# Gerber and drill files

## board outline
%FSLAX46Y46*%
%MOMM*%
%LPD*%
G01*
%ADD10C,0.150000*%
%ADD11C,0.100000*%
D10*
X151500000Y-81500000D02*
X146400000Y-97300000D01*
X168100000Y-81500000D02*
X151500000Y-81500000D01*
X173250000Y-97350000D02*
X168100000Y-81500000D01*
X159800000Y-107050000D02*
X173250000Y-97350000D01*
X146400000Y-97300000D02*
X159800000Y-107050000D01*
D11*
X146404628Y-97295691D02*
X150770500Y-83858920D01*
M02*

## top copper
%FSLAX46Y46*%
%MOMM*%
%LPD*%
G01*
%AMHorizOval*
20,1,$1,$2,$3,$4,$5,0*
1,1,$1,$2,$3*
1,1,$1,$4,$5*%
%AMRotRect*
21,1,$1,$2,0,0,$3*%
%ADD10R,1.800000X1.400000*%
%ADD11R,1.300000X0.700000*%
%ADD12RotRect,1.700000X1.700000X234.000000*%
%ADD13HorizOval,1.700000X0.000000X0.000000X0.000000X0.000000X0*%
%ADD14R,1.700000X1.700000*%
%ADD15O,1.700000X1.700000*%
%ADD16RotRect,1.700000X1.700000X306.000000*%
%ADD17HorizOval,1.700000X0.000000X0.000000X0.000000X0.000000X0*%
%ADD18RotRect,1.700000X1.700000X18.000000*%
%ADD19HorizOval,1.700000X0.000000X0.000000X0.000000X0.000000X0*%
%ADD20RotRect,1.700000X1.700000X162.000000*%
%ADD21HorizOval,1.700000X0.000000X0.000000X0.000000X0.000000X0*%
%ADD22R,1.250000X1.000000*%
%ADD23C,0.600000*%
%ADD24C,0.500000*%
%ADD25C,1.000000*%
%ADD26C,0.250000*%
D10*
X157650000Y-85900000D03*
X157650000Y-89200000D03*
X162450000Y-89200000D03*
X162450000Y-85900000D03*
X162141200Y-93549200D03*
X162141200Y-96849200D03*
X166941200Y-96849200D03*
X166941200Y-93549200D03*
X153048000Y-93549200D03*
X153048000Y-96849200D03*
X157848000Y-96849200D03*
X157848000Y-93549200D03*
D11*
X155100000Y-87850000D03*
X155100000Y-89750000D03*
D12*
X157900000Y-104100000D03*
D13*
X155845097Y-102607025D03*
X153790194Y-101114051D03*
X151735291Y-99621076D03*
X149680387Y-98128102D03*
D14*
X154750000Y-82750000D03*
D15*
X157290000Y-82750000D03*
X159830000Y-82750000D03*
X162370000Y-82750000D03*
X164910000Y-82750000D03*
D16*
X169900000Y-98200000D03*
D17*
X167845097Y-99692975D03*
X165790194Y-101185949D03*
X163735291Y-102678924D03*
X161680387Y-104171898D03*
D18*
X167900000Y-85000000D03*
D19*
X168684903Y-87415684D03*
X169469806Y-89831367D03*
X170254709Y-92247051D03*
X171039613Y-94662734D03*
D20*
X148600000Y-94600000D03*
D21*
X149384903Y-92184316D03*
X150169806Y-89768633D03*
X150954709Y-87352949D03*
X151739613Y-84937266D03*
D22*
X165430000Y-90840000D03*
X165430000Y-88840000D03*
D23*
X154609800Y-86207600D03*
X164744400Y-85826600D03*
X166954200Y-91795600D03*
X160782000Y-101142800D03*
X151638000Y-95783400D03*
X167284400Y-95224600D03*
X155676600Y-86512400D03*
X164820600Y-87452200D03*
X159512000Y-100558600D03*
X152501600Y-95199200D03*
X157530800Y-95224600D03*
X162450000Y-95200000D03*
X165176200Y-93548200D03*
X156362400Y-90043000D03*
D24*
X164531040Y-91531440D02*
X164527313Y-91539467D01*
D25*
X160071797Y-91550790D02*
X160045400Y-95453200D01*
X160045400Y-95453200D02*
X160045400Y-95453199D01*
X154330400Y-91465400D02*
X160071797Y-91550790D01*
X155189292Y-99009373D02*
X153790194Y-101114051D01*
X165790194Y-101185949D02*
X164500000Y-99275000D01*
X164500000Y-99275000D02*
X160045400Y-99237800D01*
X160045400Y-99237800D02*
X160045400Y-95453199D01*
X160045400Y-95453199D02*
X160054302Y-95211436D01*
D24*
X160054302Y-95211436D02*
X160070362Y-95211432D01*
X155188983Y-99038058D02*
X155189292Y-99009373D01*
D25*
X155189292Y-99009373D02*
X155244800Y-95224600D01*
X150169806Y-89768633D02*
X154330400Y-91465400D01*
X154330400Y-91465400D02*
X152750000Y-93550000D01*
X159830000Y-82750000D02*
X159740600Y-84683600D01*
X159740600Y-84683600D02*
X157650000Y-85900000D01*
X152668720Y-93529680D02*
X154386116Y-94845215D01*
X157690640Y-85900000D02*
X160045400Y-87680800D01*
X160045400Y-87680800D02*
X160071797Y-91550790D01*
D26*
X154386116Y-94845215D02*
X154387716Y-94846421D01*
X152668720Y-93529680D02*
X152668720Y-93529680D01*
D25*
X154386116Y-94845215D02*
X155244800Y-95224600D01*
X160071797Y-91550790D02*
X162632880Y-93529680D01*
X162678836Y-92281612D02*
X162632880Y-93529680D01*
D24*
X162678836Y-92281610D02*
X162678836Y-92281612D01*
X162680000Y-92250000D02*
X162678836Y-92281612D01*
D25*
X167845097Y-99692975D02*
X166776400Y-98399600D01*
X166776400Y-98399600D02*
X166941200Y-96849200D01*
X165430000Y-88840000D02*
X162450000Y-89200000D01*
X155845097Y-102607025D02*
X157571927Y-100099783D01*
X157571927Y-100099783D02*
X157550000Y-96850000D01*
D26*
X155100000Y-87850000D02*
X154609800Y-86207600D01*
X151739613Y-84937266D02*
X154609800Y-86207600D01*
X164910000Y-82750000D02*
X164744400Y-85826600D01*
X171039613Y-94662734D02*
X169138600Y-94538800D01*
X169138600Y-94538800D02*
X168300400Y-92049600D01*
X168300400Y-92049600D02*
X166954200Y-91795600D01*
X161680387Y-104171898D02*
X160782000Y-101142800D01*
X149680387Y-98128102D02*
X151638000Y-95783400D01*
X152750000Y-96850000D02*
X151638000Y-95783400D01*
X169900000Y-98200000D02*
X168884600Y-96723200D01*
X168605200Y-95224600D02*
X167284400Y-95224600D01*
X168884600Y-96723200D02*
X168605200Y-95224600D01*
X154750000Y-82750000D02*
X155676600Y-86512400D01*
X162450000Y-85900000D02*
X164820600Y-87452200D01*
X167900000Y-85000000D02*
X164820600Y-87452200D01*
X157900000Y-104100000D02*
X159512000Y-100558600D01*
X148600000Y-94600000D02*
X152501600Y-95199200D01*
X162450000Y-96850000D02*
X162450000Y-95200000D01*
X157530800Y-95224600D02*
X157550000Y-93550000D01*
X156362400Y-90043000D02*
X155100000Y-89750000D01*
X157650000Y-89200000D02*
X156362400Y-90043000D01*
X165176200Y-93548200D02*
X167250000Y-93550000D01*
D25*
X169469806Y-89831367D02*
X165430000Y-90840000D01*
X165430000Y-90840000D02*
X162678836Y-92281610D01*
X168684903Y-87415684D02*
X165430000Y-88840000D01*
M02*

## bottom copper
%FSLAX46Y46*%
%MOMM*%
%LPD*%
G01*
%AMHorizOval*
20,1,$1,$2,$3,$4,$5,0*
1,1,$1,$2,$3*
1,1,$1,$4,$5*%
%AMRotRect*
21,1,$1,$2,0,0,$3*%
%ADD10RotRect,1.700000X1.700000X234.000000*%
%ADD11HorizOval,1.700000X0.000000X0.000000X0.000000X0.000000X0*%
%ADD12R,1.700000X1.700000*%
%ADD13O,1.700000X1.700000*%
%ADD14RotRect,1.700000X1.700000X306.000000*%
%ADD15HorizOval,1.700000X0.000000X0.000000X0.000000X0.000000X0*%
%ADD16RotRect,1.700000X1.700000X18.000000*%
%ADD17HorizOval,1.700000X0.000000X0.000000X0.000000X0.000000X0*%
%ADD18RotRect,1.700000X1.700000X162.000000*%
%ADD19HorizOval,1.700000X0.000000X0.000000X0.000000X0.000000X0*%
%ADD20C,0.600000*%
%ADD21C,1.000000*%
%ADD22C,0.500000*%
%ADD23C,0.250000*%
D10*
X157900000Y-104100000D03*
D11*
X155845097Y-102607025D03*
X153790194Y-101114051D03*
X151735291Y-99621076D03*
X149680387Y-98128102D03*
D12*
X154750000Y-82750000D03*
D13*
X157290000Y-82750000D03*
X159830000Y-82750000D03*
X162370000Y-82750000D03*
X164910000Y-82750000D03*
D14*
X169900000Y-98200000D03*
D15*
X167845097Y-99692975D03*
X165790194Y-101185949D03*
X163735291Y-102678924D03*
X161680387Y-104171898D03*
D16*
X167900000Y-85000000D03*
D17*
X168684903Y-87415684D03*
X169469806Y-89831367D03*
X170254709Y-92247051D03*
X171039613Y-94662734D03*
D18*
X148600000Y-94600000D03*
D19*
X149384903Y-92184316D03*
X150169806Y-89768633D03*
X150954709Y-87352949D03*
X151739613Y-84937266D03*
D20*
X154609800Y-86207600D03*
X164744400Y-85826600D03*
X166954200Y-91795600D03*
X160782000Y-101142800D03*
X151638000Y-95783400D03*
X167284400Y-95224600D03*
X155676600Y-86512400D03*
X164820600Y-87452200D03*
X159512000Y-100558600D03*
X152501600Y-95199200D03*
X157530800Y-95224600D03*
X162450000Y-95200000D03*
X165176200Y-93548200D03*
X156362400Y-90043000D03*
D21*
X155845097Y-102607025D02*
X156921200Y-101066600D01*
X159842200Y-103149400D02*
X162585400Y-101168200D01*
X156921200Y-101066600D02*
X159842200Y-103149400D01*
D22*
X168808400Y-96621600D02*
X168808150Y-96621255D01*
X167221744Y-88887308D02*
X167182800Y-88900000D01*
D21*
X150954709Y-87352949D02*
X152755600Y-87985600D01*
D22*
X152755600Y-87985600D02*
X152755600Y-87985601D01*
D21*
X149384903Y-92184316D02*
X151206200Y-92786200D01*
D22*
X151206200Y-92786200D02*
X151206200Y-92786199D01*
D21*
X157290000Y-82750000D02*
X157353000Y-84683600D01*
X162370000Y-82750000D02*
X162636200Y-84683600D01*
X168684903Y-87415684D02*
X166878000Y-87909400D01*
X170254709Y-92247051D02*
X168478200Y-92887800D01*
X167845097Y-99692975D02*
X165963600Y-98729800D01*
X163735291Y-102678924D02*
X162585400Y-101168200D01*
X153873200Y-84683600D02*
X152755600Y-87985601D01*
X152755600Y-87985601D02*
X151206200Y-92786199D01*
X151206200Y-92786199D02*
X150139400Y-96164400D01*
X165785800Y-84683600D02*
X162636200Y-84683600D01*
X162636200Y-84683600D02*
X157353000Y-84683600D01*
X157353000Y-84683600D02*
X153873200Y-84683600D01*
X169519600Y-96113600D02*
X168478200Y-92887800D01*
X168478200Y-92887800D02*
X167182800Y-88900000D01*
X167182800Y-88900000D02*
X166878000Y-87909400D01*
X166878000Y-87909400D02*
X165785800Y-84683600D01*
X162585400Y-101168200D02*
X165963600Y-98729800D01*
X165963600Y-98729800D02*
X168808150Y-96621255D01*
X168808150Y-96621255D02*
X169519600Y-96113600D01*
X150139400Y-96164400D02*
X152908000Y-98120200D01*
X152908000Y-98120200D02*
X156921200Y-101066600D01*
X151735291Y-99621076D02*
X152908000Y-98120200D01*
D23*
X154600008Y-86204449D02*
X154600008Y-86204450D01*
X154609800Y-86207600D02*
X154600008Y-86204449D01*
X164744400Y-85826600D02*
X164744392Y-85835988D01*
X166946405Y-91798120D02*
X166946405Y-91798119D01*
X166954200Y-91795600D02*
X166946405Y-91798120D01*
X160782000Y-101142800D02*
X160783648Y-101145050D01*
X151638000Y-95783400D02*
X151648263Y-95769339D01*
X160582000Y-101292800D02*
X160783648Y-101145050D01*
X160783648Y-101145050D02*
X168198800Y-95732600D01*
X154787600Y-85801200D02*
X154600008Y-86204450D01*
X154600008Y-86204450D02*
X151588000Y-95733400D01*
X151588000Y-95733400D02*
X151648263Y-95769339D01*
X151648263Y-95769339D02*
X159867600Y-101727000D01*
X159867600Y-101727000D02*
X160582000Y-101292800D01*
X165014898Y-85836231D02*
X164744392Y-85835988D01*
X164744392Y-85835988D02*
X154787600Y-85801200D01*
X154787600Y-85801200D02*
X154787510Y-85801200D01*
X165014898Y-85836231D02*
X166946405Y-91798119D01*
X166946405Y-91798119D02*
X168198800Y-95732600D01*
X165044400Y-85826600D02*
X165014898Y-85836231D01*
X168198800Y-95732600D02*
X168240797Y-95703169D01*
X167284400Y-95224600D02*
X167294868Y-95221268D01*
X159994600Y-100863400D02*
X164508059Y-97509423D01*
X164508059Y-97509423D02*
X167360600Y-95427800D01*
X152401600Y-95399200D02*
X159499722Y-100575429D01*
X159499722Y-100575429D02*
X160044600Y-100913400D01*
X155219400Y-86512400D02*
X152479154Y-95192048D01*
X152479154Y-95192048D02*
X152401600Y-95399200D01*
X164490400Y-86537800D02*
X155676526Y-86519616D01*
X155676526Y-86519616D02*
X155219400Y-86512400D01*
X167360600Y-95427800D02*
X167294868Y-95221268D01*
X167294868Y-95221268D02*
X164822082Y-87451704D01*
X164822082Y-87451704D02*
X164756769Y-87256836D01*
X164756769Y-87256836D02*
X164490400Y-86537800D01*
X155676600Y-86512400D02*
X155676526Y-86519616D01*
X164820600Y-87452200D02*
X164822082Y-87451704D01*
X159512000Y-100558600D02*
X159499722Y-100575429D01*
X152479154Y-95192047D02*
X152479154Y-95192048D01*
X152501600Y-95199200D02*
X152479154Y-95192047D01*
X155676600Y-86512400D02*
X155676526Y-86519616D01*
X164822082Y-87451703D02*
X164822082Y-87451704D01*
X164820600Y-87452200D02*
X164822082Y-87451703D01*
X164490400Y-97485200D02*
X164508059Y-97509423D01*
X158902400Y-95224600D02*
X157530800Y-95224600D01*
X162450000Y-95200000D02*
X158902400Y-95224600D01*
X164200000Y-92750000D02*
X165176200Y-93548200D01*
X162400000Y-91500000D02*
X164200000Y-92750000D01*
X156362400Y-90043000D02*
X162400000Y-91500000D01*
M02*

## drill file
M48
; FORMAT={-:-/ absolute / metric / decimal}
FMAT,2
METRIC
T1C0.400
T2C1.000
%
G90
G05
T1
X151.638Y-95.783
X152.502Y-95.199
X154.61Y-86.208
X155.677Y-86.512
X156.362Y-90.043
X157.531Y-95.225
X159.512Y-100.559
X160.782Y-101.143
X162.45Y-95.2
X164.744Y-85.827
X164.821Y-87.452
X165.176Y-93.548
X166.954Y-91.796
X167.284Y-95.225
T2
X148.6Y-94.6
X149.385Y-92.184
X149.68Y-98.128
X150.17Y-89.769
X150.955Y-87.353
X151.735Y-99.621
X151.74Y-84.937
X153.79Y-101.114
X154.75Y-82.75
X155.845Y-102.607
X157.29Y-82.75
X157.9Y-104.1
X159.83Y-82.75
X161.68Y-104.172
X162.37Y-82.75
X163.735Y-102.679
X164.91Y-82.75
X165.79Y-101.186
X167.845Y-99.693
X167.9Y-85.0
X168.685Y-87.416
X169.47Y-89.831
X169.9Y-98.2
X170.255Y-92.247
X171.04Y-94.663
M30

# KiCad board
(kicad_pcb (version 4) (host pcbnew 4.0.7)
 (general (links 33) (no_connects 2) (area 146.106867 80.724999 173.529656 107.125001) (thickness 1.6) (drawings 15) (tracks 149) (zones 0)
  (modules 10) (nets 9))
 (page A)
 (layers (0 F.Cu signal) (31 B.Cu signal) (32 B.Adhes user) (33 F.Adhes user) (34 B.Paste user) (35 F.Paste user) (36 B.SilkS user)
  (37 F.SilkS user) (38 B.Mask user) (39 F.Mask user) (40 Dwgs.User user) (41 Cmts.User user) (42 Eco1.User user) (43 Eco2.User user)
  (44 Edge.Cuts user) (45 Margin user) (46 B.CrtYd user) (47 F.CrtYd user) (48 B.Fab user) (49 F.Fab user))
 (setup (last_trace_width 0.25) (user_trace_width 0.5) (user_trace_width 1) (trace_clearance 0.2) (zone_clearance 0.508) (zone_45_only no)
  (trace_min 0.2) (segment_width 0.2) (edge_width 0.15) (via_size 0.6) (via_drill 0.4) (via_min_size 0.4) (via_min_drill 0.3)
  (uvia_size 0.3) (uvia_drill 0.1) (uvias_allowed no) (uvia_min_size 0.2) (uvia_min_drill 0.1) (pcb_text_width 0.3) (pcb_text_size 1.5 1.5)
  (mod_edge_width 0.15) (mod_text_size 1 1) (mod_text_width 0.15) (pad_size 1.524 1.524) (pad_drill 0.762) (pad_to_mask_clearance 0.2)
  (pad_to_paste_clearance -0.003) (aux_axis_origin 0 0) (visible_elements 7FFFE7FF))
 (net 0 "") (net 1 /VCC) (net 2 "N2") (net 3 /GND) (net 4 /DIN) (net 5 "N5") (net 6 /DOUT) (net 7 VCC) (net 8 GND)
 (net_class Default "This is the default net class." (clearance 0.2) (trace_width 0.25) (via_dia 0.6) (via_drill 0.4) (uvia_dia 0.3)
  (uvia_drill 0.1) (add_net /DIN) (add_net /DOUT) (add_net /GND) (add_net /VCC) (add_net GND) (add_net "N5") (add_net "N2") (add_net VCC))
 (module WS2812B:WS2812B (layer F.Cu) (at 160.05 87.55 90)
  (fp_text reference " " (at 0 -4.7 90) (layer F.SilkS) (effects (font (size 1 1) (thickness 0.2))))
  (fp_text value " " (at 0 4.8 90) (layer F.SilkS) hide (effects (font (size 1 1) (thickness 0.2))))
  (pad 1 smd rect (at 1.65 -2.4 90) (size 1.4 1.8) (layers F.Cu F.Paste F.Mask) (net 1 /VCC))
  (pad 2 smd rect (at -1.65 -2.4 90) (size 1.4 1.8) (layers F.Cu F.Paste F.Mask) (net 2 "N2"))
  (pad 3 smd rect (at -1.65 2.4 90) (size 1.4 1.8) (layers F.Cu F.Paste F.Mask) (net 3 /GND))
  (pad 4 smd rect (at 1.65 2.4 90) (size 1.4 1.8) (layers F.Cu F.Paste F.Mask) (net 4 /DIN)))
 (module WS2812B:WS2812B (layer F.Cu) (at 164.5412 95.1992 90)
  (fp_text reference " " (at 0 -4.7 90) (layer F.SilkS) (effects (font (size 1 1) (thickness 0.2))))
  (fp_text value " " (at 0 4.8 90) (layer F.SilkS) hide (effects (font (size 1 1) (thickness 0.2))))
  (pad 1 smd rect (at 1.65 -2.4 90) (size 1.4 1.8) (layers F.Cu F.Paste F.Mask) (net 1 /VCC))
  (pad 2 smd rect (at -1.65 -2.4 90) (size 1.4 1.8) (layers F.Cu F.Paste F.Mask) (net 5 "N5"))
  (pad 3 smd rect (at -1.65 2.4 90) (size 1.4 1.8) (layers F.Cu F.Paste F.Mask) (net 3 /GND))
  (pad 4 smd rect (at 1.65 2.4 90) (size 1.4 1.8) (layers F.Cu F.Paste F.Mask) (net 2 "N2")))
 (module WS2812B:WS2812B (layer F.Cu) (at 155.448 95.1992 90)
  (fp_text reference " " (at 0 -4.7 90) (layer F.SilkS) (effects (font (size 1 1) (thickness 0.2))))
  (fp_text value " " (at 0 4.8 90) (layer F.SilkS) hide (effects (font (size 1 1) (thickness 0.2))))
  (pad 1 smd rect (at 1.65 -2.4 90) (size 1.4 1.8) (layers F.Cu F.Paste F.Mask) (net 1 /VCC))
  (pad 2 smd rect (at -1.65 -2.4 90) (size 1.4 1.8) (layers F.Cu F.Paste F.Mask) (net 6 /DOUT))
  (pad 3 smd rect (at -1.65 2.4 90) (size 1.4 1.8) (layers F.Cu F.Paste F.Mask) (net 3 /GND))
  (pad 4 smd rect (at 1.65 2.4 90) (size 1.4 1.8) (layers F.Cu F.Paste F.Mask) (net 5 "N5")))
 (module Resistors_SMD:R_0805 (layer F.Cu) (at 155.1 88.8 270)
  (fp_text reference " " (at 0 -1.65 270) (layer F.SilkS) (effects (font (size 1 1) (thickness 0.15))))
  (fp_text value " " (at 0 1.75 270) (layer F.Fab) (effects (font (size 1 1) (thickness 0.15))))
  (pad 1 smd rect (at -0.95 0 270) (size 0.7 1.3) (layers F.Cu F.Paste F.Mask) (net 6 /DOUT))
  (pad 2 smd rect (at 0.95 0 270) (size 0.7 1.3) (layers F.Cu F.Paste F.Mask) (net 2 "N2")))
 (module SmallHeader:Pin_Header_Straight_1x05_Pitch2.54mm (layer F.Cu) (at 157.9 104.1 234)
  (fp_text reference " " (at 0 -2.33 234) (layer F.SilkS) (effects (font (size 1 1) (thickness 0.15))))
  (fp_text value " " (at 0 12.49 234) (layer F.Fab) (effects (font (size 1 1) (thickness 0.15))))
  (pad 1 thru_hole rect (at 0 0 234) (size 1.7 1.7) (drill 1) (layers *.Cu *.Mask) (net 4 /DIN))
  (pad 2 thru_hole oval (at 0 2.54 234) (size 1.7 1.7) (drill 1) (layers *.Cu *.Mask) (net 3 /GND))
  (pad 3 thru_hole oval (at 0 5.08 234) (size 1.7 1.7) (drill 1) (layers *.Cu *.Mask) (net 1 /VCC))
  (pad 4 thru_hole oval (at 0 7.62 234) (size 1.7 1.7) (drill 1) (layers *.Cu *.Mask) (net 3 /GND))
  (pad 5 thru_hole oval (at 0 10.16 234) (size 1.7 1.7) (drill 1) (layers *.Cu *.Mask) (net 6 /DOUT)))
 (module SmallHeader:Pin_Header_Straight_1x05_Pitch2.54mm (layer F.Cu) (at 154.75 82.75 90)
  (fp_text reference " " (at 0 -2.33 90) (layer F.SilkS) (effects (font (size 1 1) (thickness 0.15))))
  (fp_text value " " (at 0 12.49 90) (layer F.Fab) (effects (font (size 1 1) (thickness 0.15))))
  (pad 1 thru_hole rect (at 0 0 90) (size 1.7 1.7) (drill 1) (layers *.Cu *.Mask) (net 4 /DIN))
  (pad 2 thru_hole oval (at 0 2.54 90) (size 1.7 1.7) (drill 1) (layers *.Cu *.Mask) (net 3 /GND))
  (pad 3 thru_hole oval (at 0 5.08 90) (size 1.7 1.7) (drill 1) (layers *.Cu *.Mask) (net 1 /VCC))
  (pad 4 thru_hole oval (at 0 7.62 90) (size 1.7 1.7) (drill 1) (layers *.Cu *.Mask) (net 3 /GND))
  (pad 5 thru_hole oval (at 0 10.16 90) (size 1.7 1.7) (drill 1) (layers *.Cu *.Mask) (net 6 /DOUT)))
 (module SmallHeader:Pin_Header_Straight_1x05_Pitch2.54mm (layer F.Cu) (at 169.9 98.2 306)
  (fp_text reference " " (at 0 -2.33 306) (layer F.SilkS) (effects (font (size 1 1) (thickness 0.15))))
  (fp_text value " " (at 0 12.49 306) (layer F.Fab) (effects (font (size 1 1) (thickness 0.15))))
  (pad 1 thru_hole rect (at 0 0 306) (size 1.7 1.7) (drill 1) (layers *.Cu *.Mask) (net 4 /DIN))
  (pad 2 thru_hole oval (at 0 2.54 306) (size 1.7 1.7) (drill 1) (layers *.Cu *.Mask) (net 3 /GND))
  (pad 3 thru_hole oval (at 0 5.08 306) (size 1.7 1.7) (drill 1) (layers *.Cu *.Mask) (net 1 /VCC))
  (pad 4 thru_hole oval (at 0 7.62 306) (size 1.7 1.7) (drill 1) (layers *.Cu *.Mask) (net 3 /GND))
  (pad 5 thru_hole oval (at 0 10.16 306) (size 1.7 1.7) (drill 1) (layers *.Cu *.Mask) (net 6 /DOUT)))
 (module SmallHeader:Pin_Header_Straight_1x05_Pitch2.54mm (layer F.Cu) (at 167.9 85 18)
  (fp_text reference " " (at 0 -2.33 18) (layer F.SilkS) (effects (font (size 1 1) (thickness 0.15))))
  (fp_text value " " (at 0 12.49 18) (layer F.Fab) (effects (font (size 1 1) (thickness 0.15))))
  (pad 1 thru_hole rect (at 0 0 18) (size 1.7 1.7) (drill 1) (layers *.Cu *.Mask) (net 4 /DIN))
  (pad 2 thru_hole oval (at 0 2.54 18) (size 1.7 1.7) (drill 1) (layers *.Cu *.Mask) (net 3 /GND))
  (pad 3 thru_hole oval (at 0 5.08 18) (size 1.7 1.7) (drill 1) (layers *.Cu *.Mask) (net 1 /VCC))
  (pad 4 thru_hole oval (at 0 7.62 18) (size 1.7 1.7) (drill 1) (layers *.Cu *.Mask) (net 3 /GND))
  (pad 5 thru_hole oval (at 0 10.16 18) (size 1.7 1.7) (drill 1) (layers *.Cu *.Mask) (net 6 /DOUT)))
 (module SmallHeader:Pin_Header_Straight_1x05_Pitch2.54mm (layer F.Cu) (at 148.6 94.6 162)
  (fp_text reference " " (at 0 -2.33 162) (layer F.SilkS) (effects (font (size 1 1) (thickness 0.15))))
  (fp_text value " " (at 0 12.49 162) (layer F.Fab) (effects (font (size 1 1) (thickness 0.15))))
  (pad 1 thru_hole rect (at 0 0 162) (size 1.7 1.7) (drill 1) (layers *.Cu *.Mask) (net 4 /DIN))
  (pad 2 thru_hole oval (at 0 2.54 162) (size 1.7 1.7) (drill 1) (layers *.Cu *.Mask) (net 3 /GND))
  (pad 3 thru_hole oval (at 0 5.08 162) (size 1.7 1.7) (drill 1) (layers *.Cu *.Mask) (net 1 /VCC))
  (pad 4 thru_hole oval (at 0 7.62 162) (size 1.7 1.7) (drill 1) (layers *.Cu *.Mask) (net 3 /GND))
  (pad 5 thru_hole oval (at 0 10.16 162) (size 1.7 1.7) (drill 1) (layers *.Cu *.Mask) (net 6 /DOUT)))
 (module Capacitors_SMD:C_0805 (layer F.Cu) (at 165.43 89.84 90)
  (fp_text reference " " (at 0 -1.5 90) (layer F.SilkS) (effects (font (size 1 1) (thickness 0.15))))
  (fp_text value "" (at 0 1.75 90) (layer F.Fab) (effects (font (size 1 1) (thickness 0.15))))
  (pad 1 smd rect (at -1 0 90) (size 1 1.25) (layers F.Cu F.Paste F.Mask) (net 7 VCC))
  (pad 2 smd rect (at 1 0 90) (size 1 1.25) (layers F.Cu F.Paste F.Mask) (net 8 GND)))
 (gr_line (start 151.5 81.5) (end 146.4 97.3) (angle 90) (layer Edge.Cuts) (width 0.15))
 (gr_line (start 168.1 81.5) (end 151.5 81.5) (angle 90) (layer Edge.Cuts) (width 0.15))
 (gr_line (start 173.25 97.35) (end 168.1 81.5) (angle 90) (layer Edge.Cuts) (width 0.15))
 (gr_line (start 159.8 107.05) (end 173.25 97.35) (angle 90) (layer Edge.Cuts) (width 0.15))
 (gr_line (start 146.4 97.3) (end 159.8 107.05) (angle 90) (layer Edge.Cuts) (width 0.15))
 (gr_line (start 146.404628 97.295691) (end 150.7705 83.85892) (layer Edge.Cuts) (width 0.1))
 (segment (start 164.53104 91.53144) (end 164.527313 91.539467) (width 0.5) (layer F.Cu) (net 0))
 (segment (start 160.071797 91.55079) (end 160.0454 95.4532) (width 1) (layer F.Cu) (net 1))
 (segment (start 160.0454 95.4532) (end 160.0454 95.453199) (width 1) (layer F.Cu) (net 1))
 (segment (start 154.3304 91.4654) (end 160.071797 91.55079) (width 1) (layer F.Cu) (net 1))
 (segment (start 155.189292 99.009373) (end 153.790194 101.114051) (width 1) (layer F.Cu) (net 1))
 (segment (start 165.790194 101.185949) (end 164.5 99.275) (width 1) (layer F.Cu) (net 1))
 (segment (start 164.5 99.275) (end 160.0454 99.2378) (width 1) (layer F.Cu) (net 1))
 (segment (start 160.0454 99.2378) (end 160.0454 95.453199) (width 1) (layer F.Cu) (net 1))
 (segment (start 160.0454 95.453199) (end 160.054302 95.211436) (width 1) (layer F.Cu) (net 1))
 (segment (start 160.054302 95.211436) (end 160.070362 95.211432) (width 0.5) (layer F.Cu) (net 1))
 (segment (start 155.188983 99.038058) (end 155.189292 99.009373) (width 0.5) (layer F.Cu) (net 1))
 (segment (start 155.189292 99.009373) (end 155.2448 95.2246) (width 1) (layer F.Cu) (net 1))
 (segment (start 150.169806 89.768633) (end 154.3304 91.4654) (width 1) (layer F.Cu) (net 1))
 (segment (start 154.3304 91.4654) (end 152.75 93.55) (width 1) (layer F.Cu) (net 1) (status 20))
 (segment (start 159.83 82.75) (end 159.7406 84.6836) (width 1) (layer F.Cu) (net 1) (status 20))
 (segment (start 159.7406 84.6836) (end 157.65 85.9) (width 1) (layer F.Cu) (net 1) (status 20))
 (segment (start 152.66872 93.52968) (end 154.386116 94.845215) (width 1) (layer F.Cu) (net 1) (status 10))
 (segment (start 157.69064 85.9) (end 160.0454 87.6808) (width 1) (layer F.Cu) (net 1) (status 10))
 (segment (start 160.0454 87.6808) (end 160.071797 91.55079) (width 1) (layer F.Cu) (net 1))
 (segment (start 154.386116 94.845215) (end 154.387716 94.846421) (width 0.25) (layer F.Cu) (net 1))
 (segment (start 152.66872 93.52968) (end 152.66872 93.52968) (width 0.25) (layer F.Cu) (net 1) (status 30))
 (segment (start 154.386116 94.845215) (end 155.2448 95.2246) (width 1) (layer F.Cu) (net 1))
 (segment (start 160.071797 91.55079) (end 162.63288 93.52968) (width 1) (layer F.Cu) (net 1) (status 20))
 (segment (start 162.678836 92.281612) (end 162.63288 93.52968) (width 1) (layer F.Cu) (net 1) (status 20))
 (segment (start 162.678836 92.28161) (end 162.678836 92.281612) (width 0.5) (layer F.Cu) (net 1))
 (segment (start 162.68 92.25) (end 162.678836 92.281612) (width 0.5) (layer F.Cu) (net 1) (status 20))
 (segment (start 167.845097 99.692975) (end 166.7764 98.3996) (width 1) (layer F.Cu) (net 3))
 (segment (start 166.7764 98.3996) (end 166.9412 96.8492) (width 1) (layer F.Cu) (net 3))
 (segment (start 155.845097 102.607025) (end 156.9212 101.0666) (width 1) (layer B.Cu) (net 3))
 (segment (start 165.43 88.84) (end 162.45 89.2) (width 1) (layer F.Cu) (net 3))
 (segment (start 159.8422 103.1494) (end 162.5854 101.1682) (width 1) (layer B.Cu) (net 3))
 (segment (start 156.9212 101.0666) (end 159.8422 103.1494) (width 1) (layer B.Cu) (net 3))
 (segment (start 155.845097 102.607025) (end 157.571927 100.099783) (width 1) (layer F.Cu) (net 3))
 (segment (start 157.571927 100.099783) (end 157.55 96.85) (width 1) (layer F.Cu) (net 3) (status 20))
 (segment (start 168.8084 96.6216) (end 168.80815 96.621255) (width 0.5) (layer B.Cu) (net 3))
 (segment (start 167.221744 88.887308) (end 167.1828 88.9) (width 0.5) (layer B.Cu) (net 3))
 (segment (start 150.954709 87.352949) (end 152.7556 87.9856) (width 1) (layer B.Cu) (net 3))
 (segment (start 152.7556 87.9856) (end 152.7556 87.985601) (width 0.5) (layer B.Cu) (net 3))
 (segment (start 149.384903 92.184316) (end 151.2062 92.7862) (width 1) (layer B.Cu) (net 3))
 (segment (start 151.2062 92.7862) (end 151.2062 92.786199) (width 0.5) (layer B.Cu) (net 3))
 (segment (start 157.29 82.75) (end 157.353 84.6836) (width 1) (layer B.Cu) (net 3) (status 10))
 (segment (start 162.37 82.75) (end 162.6362 84.6836) (width 1) (layer B.Cu) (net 3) (status 10))
 (segment (start 168.684903 87.415684) (end 166.878 87.9094) (width 1) (layer B.Cu) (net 3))
 (segment (start 170.254709 92.247051) (end 168.4782 92.8878) (width 1) (layer B.Cu) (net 3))
 (segment (start 167.845097 99.692975) (end 165.9636 98.7298) (width 1) (layer B.Cu) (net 3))
 (segment (start 163.735291 102.678924) (end 162.5854 101.1682) (width 1) (layer B.Cu) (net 3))
 (segment (start 153.8732 84.6836) (end 152.7556 87.985601) (width 1) (layer B.Cu) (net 3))
 (segment (start 152.7556 87.985601) (end 151.2062 92.786199) (width 1) (layer B.Cu) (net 3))
 (segment (start 151.2062 92.786199) (end 150.1394 96.1644) (width 1) (layer B.Cu) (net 3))
 (segment (start 165.7858 84.6836) (end 162.6362 84.6836) (width 1) (layer B.Cu) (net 3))
 (segment (start 162.6362 84.6836) (end 157.353 84.6836) (width 1) (layer B.Cu) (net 3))
 (segment (start 157.353 84.6836) (end 153.8732 84.6836) (width 1) (layer B.Cu) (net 3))
 (segment (start 169.5196 96.1136) (end 168.4782 92.8878) (width 1) (layer B.Cu) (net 3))
 (segment (start 168.4782 92.8878) (end 167.1828 88.9) (width 1) (layer B.Cu) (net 3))
 (segment (start 167.1828 88.9) (end 166.878 87.9094) (width 1) (layer B.Cu) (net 3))
 (segment (start 166.878 87.9094) (end 165.7858 84.6836) (width 1) (layer B.Cu) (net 3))
 (segment (start 162.5854 101.1682) (end 165.9636 98.7298) (width 1) (layer B.Cu) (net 3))
 (segment (start 165.9636 98.7298) (end 168.80815 96.621255) (width 1) (layer B.Cu) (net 3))
 (segment (start 168.80815 96.621255) (end 169.5196 96.1136) (width 1) (layer B.Cu) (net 3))
 (segment (start 150.1394 96.1644) (end 152.908 98.1202) (width 1) (layer B.Cu) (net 3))
 (segment (start 152.908 98.1202) (end 156.9212 101.0666) (width 1) (layer B.Cu) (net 3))
 (segment (start 151.735291 99.621076) (end 152.908 98.1202) (width 1) (layer B.Cu) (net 3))
 (segment (start 155.1 87.85) (end 154.6098 86.2076) (width 0.25) (layer F.Cu) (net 6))
 (segment (start 151.739613 84.937266) (end 154.6098 86.2076) (width 0.25) (layer F.Cu) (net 6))
 (segment (start 154.600008 86.204449) (end 154.600008 86.20445) (width 0.25) (layer B.Cu) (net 6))
 (segment (start 154.6098 86.2076) (end 154.600008 86.204449) (width 0.25) (layer B.Cu) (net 6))
 (via (at 154.6098 86.2076) (size 0.6) (drill 0.4) (layers F.Cu B.Cu) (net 6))
 (segment (start 164.91 82.75) (end 164.7444 85.8266) (width 0.25) (layer F.Cu) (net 6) (status 10))
 (segment (start 164.7444 85.8266) (end 164.744392 85.835988) (width 0.25) (layer B.Cu) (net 6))
 (via (at 164.7444 85.8266) (size 0.6) (drill 0.4) (layers F.Cu B.Cu) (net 6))
 (segment (start 171.039613 94.662734) (end 169.1386 94.5388) (width 0.25) (layer F.Cu) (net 6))
 (segment (start 169.1386 94.5388) (end 168.3004 92.0496) (width 0.25) (layer F.Cu) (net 6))
 (segment (start 168.3004 92.0496) (end 166.9542 91.7956) (width 0.25) (layer F.Cu) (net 6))
 (segment (start 166.946405 91.79812) (end 166.946405 91.798119) (width 0.25) (layer B.Cu) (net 6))
 (segment (start 166.9542 91.7956) (end 166.946405 91.79812) (width 0.25) (layer B.Cu) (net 6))
 (via (at 166.9542 91.7956) (size 0.6) (drill 0.4) (layers F.Cu B.Cu) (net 6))
 (segment (start 161.680387 104.171898) (end 160.782 101.1428) (width 0.25) (layer F.Cu) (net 6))
 (segment (start 160.782 101.1428) (end 160.783648 101.14505) (width 0.25) (layer B.Cu) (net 6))
 (via (at 160.782 101.1428) (size 0.6) (drill 0.4) (layers F.Cu B.Cu) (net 6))
 (segment (start 149.680387 98.128102) (end 151.638 95.7834) (width 0.25) (layer F.Cu) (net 6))
 (segment (start 152.75 96.85) (end 151.638 95.7834) (width 0.25) (layer F.Cu) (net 6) (status 10))
 (segment (start 151.638 95.7834) (end 151.648263 95.769339) (width 0.25) (layer B.Cu) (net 6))
 (via (at 151.638 95.7834) (size 0.6) (drill 0.4) (layers F.Cu B.Cu) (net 6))
 (segment (start 160.582 101.2928) (end 160.783648 101.14505) (width 0.25) (layer B.Cu) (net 6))
 (segment (start 160.783648 101.14505) (end 168.1988 95.7326) (width 0.25) (layer B.Cu) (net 6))
 (segment (start 154.7876 85.8012) (end 154.600008 86.20445) (width 0.25) (layer B.Cu) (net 6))
 (segment (start 154.600008 86.20445) (end 151.588 95.7334) (width 0.25) (layer B.Cu) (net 6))
 (segment (start 151.588 95.7334) (end 151.648263 95.769339) (width 0.25) (layer B.Cu) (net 6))
 (segment (start 151.648263 95.769339) (end 159.8676 101.727) (width 0.25) (layer B.Cu) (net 6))
 (segment (start 159.8676 101.727) (end 160.582 101.2928) (width 0.25) (layer B.Cu) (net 6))
 (segment (start 165.014898 85.836231) (end 164.744392 85.835988) (width 0.25) (layer B.Cu) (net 6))
 (segment (start 164.744392 85.835988) (end 154.7876 85.8012) (width 0.25) (layer B.Cu) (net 6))
 (segment (start 154.7876 85.8012) (end 154.78751 85.8012) (width 0.25) (layer B.Cu) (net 6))
 (segment (start 165.014898 85.836231) (end 166.946405 91.798119) (width 0.25) (layer B.Cu) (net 6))
 (segment (start 166.946405 91.798119) (end 168.1988 95.7326) (width 0.25) (layer B.Cu) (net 6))
 (segment (start 165.0444 85.8266) (end 165.014898 85.836231) (width 0.25) (layer B.Cu) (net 6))
 (segment (start 168.1988 95.7326) (end 168.240797 95.703169) (width 0.25) (layer B.Cu) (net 6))
 (segment (start 169.9 98.2) (end 168.8846 96.7232) (width 0.25) (layer F.Cu) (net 4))
 (segment (start 167.2844 95.2246) (end 167.294868 95.221268) (width 0.25) (layer B.Cu) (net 4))
 (via (at 167.2844 95.2246) (size 0.6) (drill 0.4) (layers F.Cu B.Cu) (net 4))
 (segment (start 168.6052 95.2246) (end 167.2844 95.2246) (width 0.25) (layer F.Cu) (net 4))
 (segment (start 168.8846 96.7232) (end 168.6052 95.2246) (width 0.25) (layer F.Cu) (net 4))
 (segment (start 159.9946 100.8634) (end 164.508059 97.509423) (width 0.25) (layer B.Cu) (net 4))
 (segment (start 164.508059 97.509423) (end 167.3606 95.4278) (width 0.25) (layer B.Cu) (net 4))
 (segment (start 152.4016 95.3992) (end 159.499722 100.575429) (width 0.25) (layer B.Cu) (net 4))
 (segment (start 159.499722 100.575429) (end 160.0446 100.9134) (width 0.25) (layer B.Cu) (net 4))
 (segment (start 155.2194 86.5124) (end 152.479154 95.192048) (width 0.25) (layer B.Cu) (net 4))
 (segment (start 152.479154 95.192048) (end 152.4016 95.3992) (width 0.25) (layer B.Cu) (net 4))
 (segment (start 164.4904 86.5378) (end 155.676526 86.519616) (width 0.25) (layer B.Cu) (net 4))
 (segment (start 155.676526 86.519616) (end 155.2194 86.5124) (width 0.25) (layer B.Cu) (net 4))
 (segment (start 167.3606 95.4278) (end 167.294868 95.221268) (width 0.25) (layer B.Cu) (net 4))
 (segment (start 167.294868 95.221268) (end 164.822082 87.451704) (width 0.25) (layer B.Cu) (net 4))
 (segment (start 164.822082 87.451704) (end 164.756769 87.256836) (width 0.25) (layer B.Cu) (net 4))
 (segment (start 164.756769 87.256836) (end 164.4904 86.5378) (width 0.25) (layer B.Cu) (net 4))
 (segment (start 154.75 82.75) (end 155.6766 86.5124) (width 0.25) (layer F.Cu) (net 4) (status 10))
 (via (at 155.6766 86.5124) (size 0.6) (drill 0.4) (layers F.Cu B.Cu) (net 4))
 (segment (start 155.6766 86.5124) (end 155.676526 86.519616) (width 0.25) (layer B.Cu) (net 4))
 (segment (start 162.45 85.9) (end 164.8206 87.4522) (width 0.25) (layer F.Cu) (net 4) (status 10))
 (segment (start 167.9 85) (end 164.8206 87.4522) (width 0.25) (layer F.Cu) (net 4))
 (via (at 164.8206 87.4522) (size 0.6) (drill 0.4) (layers F.Cu B.Cu) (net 4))
 (segment (start 164.8206 87.4522) (end 164.822082 87.451704) (width 0.25) (layer B.Cu) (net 4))
 (segment (start 157.9 104.1) (end 159.512 100.5586) (width 0.25) (layer F.Cu) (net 4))
 (segment (start 159.512 100.5586) (end 159.499722 100.575429) (width 0.25) (layer B.Cu) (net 4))
 (via (at 159.512 100.5586) (size 0.6) (drill 0.4) (layers F.Cu B.Cu) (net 4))
 (segment (start 148.6 94.6) (end 152.5016 95.1992) (width 0.25) (layer F.Cu) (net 4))
 (segment (start 152.479154 95.192047) (end 152.479154 95.192048) (width 0.25) (layer B.Cu) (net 4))
 (segment (start 152.5016 95.1992) (end 152.479154 95.192047) (width 0.25) (layer B.Cu) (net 4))
 (via (at 152.5016 95.1992) (size 0.6) (drill 0.4) (layers F.Cu B.Cu) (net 4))
 (segment (start 155.6766 86.5124) (end 155.676526 86.519616) (width 0.25) (layer B.Cu) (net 4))
 (segment (start 164.822082 87.451703) (end 164.822082 87.451704) (width 0.25) (layer B.Cu) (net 4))
 (segment (start 164.8206 87.4522) (end 164.822082 87.451703) (width 0.25) (layer B.Cu) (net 4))
 (segment (start 164.4904 97.4852) (end 164.508059 97.509423) (width 0.25) (layer B.Cu) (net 4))
 (segment (start 162.45 96.85) (end 162.45 95.2) (width 0.25) (layer F.Cu) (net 5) (status 10))
 (segment (start 157.5308 95.2246) (end 157.55 93.55) (width 0.25) (layer F.Cu) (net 5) (status 20))
 (via (at 157.5308 95.2246) (size 0.6) (drill 0.4) (layers F.Cu B.Cu) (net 5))
 (segment (start 158.9024 95.2246) (end 157.5308 95.2246) (width 0.25) (layer B.Cu) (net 5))
 (segment (start 162.45 95.2) (end 158.9024 95.2246) (width 0.25) (layer B.Cu) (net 5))
 (via (at 162.45 95.2) (size 0.6) (drill 0.4) (layers F.Cu B.Cu) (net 5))
 (segment (start 156.3624 90.043) (end 155.1 89.75) (width 0.25) (layer F.Cu) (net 2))
 (segment (start 157.65 89.2) (end 156.3624 90.043) (width 0.25) (layer F.Cu) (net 2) (status 10))
 (segment (start 165.1762 93.5482) (end 167.25 93.55) (width 0.25) (layer F.Cu) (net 2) (status 20))
 (via (at 165.1762 93.5482) (size 0.6) (drill 0.4) (layers F.Cu B.Cu) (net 2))
 (segment (start 164.2 92.75) (end 165.1762 93.5482) (width 0.25) (layer B.Cu) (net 2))
 (segment (start 162.4 91.5) (end 164.2 92.75) (width 0.25) (layer B.Cu) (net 2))
 (segment (start 156.3624 90.043) (end 162.4 91.5) (width 0.25) (layer B.Cu) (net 2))
 (via (at 156.3624 90.043) (size 0.6) (drill 0.4) (layers F.Cu B.Cu) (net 2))
 (segment (start 169.469806 89.831367) (end 165.43 90.84) (width 1) (layer F.Cu) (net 7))
 (segment (start 165.43 90.84) (end 162.678836 92.28161) (width 1) (layer F.Cu) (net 7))
 (segment (start 168.684903 87.415684) (end 165.43 88.84) (width 1) (layer F.Cu) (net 8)))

